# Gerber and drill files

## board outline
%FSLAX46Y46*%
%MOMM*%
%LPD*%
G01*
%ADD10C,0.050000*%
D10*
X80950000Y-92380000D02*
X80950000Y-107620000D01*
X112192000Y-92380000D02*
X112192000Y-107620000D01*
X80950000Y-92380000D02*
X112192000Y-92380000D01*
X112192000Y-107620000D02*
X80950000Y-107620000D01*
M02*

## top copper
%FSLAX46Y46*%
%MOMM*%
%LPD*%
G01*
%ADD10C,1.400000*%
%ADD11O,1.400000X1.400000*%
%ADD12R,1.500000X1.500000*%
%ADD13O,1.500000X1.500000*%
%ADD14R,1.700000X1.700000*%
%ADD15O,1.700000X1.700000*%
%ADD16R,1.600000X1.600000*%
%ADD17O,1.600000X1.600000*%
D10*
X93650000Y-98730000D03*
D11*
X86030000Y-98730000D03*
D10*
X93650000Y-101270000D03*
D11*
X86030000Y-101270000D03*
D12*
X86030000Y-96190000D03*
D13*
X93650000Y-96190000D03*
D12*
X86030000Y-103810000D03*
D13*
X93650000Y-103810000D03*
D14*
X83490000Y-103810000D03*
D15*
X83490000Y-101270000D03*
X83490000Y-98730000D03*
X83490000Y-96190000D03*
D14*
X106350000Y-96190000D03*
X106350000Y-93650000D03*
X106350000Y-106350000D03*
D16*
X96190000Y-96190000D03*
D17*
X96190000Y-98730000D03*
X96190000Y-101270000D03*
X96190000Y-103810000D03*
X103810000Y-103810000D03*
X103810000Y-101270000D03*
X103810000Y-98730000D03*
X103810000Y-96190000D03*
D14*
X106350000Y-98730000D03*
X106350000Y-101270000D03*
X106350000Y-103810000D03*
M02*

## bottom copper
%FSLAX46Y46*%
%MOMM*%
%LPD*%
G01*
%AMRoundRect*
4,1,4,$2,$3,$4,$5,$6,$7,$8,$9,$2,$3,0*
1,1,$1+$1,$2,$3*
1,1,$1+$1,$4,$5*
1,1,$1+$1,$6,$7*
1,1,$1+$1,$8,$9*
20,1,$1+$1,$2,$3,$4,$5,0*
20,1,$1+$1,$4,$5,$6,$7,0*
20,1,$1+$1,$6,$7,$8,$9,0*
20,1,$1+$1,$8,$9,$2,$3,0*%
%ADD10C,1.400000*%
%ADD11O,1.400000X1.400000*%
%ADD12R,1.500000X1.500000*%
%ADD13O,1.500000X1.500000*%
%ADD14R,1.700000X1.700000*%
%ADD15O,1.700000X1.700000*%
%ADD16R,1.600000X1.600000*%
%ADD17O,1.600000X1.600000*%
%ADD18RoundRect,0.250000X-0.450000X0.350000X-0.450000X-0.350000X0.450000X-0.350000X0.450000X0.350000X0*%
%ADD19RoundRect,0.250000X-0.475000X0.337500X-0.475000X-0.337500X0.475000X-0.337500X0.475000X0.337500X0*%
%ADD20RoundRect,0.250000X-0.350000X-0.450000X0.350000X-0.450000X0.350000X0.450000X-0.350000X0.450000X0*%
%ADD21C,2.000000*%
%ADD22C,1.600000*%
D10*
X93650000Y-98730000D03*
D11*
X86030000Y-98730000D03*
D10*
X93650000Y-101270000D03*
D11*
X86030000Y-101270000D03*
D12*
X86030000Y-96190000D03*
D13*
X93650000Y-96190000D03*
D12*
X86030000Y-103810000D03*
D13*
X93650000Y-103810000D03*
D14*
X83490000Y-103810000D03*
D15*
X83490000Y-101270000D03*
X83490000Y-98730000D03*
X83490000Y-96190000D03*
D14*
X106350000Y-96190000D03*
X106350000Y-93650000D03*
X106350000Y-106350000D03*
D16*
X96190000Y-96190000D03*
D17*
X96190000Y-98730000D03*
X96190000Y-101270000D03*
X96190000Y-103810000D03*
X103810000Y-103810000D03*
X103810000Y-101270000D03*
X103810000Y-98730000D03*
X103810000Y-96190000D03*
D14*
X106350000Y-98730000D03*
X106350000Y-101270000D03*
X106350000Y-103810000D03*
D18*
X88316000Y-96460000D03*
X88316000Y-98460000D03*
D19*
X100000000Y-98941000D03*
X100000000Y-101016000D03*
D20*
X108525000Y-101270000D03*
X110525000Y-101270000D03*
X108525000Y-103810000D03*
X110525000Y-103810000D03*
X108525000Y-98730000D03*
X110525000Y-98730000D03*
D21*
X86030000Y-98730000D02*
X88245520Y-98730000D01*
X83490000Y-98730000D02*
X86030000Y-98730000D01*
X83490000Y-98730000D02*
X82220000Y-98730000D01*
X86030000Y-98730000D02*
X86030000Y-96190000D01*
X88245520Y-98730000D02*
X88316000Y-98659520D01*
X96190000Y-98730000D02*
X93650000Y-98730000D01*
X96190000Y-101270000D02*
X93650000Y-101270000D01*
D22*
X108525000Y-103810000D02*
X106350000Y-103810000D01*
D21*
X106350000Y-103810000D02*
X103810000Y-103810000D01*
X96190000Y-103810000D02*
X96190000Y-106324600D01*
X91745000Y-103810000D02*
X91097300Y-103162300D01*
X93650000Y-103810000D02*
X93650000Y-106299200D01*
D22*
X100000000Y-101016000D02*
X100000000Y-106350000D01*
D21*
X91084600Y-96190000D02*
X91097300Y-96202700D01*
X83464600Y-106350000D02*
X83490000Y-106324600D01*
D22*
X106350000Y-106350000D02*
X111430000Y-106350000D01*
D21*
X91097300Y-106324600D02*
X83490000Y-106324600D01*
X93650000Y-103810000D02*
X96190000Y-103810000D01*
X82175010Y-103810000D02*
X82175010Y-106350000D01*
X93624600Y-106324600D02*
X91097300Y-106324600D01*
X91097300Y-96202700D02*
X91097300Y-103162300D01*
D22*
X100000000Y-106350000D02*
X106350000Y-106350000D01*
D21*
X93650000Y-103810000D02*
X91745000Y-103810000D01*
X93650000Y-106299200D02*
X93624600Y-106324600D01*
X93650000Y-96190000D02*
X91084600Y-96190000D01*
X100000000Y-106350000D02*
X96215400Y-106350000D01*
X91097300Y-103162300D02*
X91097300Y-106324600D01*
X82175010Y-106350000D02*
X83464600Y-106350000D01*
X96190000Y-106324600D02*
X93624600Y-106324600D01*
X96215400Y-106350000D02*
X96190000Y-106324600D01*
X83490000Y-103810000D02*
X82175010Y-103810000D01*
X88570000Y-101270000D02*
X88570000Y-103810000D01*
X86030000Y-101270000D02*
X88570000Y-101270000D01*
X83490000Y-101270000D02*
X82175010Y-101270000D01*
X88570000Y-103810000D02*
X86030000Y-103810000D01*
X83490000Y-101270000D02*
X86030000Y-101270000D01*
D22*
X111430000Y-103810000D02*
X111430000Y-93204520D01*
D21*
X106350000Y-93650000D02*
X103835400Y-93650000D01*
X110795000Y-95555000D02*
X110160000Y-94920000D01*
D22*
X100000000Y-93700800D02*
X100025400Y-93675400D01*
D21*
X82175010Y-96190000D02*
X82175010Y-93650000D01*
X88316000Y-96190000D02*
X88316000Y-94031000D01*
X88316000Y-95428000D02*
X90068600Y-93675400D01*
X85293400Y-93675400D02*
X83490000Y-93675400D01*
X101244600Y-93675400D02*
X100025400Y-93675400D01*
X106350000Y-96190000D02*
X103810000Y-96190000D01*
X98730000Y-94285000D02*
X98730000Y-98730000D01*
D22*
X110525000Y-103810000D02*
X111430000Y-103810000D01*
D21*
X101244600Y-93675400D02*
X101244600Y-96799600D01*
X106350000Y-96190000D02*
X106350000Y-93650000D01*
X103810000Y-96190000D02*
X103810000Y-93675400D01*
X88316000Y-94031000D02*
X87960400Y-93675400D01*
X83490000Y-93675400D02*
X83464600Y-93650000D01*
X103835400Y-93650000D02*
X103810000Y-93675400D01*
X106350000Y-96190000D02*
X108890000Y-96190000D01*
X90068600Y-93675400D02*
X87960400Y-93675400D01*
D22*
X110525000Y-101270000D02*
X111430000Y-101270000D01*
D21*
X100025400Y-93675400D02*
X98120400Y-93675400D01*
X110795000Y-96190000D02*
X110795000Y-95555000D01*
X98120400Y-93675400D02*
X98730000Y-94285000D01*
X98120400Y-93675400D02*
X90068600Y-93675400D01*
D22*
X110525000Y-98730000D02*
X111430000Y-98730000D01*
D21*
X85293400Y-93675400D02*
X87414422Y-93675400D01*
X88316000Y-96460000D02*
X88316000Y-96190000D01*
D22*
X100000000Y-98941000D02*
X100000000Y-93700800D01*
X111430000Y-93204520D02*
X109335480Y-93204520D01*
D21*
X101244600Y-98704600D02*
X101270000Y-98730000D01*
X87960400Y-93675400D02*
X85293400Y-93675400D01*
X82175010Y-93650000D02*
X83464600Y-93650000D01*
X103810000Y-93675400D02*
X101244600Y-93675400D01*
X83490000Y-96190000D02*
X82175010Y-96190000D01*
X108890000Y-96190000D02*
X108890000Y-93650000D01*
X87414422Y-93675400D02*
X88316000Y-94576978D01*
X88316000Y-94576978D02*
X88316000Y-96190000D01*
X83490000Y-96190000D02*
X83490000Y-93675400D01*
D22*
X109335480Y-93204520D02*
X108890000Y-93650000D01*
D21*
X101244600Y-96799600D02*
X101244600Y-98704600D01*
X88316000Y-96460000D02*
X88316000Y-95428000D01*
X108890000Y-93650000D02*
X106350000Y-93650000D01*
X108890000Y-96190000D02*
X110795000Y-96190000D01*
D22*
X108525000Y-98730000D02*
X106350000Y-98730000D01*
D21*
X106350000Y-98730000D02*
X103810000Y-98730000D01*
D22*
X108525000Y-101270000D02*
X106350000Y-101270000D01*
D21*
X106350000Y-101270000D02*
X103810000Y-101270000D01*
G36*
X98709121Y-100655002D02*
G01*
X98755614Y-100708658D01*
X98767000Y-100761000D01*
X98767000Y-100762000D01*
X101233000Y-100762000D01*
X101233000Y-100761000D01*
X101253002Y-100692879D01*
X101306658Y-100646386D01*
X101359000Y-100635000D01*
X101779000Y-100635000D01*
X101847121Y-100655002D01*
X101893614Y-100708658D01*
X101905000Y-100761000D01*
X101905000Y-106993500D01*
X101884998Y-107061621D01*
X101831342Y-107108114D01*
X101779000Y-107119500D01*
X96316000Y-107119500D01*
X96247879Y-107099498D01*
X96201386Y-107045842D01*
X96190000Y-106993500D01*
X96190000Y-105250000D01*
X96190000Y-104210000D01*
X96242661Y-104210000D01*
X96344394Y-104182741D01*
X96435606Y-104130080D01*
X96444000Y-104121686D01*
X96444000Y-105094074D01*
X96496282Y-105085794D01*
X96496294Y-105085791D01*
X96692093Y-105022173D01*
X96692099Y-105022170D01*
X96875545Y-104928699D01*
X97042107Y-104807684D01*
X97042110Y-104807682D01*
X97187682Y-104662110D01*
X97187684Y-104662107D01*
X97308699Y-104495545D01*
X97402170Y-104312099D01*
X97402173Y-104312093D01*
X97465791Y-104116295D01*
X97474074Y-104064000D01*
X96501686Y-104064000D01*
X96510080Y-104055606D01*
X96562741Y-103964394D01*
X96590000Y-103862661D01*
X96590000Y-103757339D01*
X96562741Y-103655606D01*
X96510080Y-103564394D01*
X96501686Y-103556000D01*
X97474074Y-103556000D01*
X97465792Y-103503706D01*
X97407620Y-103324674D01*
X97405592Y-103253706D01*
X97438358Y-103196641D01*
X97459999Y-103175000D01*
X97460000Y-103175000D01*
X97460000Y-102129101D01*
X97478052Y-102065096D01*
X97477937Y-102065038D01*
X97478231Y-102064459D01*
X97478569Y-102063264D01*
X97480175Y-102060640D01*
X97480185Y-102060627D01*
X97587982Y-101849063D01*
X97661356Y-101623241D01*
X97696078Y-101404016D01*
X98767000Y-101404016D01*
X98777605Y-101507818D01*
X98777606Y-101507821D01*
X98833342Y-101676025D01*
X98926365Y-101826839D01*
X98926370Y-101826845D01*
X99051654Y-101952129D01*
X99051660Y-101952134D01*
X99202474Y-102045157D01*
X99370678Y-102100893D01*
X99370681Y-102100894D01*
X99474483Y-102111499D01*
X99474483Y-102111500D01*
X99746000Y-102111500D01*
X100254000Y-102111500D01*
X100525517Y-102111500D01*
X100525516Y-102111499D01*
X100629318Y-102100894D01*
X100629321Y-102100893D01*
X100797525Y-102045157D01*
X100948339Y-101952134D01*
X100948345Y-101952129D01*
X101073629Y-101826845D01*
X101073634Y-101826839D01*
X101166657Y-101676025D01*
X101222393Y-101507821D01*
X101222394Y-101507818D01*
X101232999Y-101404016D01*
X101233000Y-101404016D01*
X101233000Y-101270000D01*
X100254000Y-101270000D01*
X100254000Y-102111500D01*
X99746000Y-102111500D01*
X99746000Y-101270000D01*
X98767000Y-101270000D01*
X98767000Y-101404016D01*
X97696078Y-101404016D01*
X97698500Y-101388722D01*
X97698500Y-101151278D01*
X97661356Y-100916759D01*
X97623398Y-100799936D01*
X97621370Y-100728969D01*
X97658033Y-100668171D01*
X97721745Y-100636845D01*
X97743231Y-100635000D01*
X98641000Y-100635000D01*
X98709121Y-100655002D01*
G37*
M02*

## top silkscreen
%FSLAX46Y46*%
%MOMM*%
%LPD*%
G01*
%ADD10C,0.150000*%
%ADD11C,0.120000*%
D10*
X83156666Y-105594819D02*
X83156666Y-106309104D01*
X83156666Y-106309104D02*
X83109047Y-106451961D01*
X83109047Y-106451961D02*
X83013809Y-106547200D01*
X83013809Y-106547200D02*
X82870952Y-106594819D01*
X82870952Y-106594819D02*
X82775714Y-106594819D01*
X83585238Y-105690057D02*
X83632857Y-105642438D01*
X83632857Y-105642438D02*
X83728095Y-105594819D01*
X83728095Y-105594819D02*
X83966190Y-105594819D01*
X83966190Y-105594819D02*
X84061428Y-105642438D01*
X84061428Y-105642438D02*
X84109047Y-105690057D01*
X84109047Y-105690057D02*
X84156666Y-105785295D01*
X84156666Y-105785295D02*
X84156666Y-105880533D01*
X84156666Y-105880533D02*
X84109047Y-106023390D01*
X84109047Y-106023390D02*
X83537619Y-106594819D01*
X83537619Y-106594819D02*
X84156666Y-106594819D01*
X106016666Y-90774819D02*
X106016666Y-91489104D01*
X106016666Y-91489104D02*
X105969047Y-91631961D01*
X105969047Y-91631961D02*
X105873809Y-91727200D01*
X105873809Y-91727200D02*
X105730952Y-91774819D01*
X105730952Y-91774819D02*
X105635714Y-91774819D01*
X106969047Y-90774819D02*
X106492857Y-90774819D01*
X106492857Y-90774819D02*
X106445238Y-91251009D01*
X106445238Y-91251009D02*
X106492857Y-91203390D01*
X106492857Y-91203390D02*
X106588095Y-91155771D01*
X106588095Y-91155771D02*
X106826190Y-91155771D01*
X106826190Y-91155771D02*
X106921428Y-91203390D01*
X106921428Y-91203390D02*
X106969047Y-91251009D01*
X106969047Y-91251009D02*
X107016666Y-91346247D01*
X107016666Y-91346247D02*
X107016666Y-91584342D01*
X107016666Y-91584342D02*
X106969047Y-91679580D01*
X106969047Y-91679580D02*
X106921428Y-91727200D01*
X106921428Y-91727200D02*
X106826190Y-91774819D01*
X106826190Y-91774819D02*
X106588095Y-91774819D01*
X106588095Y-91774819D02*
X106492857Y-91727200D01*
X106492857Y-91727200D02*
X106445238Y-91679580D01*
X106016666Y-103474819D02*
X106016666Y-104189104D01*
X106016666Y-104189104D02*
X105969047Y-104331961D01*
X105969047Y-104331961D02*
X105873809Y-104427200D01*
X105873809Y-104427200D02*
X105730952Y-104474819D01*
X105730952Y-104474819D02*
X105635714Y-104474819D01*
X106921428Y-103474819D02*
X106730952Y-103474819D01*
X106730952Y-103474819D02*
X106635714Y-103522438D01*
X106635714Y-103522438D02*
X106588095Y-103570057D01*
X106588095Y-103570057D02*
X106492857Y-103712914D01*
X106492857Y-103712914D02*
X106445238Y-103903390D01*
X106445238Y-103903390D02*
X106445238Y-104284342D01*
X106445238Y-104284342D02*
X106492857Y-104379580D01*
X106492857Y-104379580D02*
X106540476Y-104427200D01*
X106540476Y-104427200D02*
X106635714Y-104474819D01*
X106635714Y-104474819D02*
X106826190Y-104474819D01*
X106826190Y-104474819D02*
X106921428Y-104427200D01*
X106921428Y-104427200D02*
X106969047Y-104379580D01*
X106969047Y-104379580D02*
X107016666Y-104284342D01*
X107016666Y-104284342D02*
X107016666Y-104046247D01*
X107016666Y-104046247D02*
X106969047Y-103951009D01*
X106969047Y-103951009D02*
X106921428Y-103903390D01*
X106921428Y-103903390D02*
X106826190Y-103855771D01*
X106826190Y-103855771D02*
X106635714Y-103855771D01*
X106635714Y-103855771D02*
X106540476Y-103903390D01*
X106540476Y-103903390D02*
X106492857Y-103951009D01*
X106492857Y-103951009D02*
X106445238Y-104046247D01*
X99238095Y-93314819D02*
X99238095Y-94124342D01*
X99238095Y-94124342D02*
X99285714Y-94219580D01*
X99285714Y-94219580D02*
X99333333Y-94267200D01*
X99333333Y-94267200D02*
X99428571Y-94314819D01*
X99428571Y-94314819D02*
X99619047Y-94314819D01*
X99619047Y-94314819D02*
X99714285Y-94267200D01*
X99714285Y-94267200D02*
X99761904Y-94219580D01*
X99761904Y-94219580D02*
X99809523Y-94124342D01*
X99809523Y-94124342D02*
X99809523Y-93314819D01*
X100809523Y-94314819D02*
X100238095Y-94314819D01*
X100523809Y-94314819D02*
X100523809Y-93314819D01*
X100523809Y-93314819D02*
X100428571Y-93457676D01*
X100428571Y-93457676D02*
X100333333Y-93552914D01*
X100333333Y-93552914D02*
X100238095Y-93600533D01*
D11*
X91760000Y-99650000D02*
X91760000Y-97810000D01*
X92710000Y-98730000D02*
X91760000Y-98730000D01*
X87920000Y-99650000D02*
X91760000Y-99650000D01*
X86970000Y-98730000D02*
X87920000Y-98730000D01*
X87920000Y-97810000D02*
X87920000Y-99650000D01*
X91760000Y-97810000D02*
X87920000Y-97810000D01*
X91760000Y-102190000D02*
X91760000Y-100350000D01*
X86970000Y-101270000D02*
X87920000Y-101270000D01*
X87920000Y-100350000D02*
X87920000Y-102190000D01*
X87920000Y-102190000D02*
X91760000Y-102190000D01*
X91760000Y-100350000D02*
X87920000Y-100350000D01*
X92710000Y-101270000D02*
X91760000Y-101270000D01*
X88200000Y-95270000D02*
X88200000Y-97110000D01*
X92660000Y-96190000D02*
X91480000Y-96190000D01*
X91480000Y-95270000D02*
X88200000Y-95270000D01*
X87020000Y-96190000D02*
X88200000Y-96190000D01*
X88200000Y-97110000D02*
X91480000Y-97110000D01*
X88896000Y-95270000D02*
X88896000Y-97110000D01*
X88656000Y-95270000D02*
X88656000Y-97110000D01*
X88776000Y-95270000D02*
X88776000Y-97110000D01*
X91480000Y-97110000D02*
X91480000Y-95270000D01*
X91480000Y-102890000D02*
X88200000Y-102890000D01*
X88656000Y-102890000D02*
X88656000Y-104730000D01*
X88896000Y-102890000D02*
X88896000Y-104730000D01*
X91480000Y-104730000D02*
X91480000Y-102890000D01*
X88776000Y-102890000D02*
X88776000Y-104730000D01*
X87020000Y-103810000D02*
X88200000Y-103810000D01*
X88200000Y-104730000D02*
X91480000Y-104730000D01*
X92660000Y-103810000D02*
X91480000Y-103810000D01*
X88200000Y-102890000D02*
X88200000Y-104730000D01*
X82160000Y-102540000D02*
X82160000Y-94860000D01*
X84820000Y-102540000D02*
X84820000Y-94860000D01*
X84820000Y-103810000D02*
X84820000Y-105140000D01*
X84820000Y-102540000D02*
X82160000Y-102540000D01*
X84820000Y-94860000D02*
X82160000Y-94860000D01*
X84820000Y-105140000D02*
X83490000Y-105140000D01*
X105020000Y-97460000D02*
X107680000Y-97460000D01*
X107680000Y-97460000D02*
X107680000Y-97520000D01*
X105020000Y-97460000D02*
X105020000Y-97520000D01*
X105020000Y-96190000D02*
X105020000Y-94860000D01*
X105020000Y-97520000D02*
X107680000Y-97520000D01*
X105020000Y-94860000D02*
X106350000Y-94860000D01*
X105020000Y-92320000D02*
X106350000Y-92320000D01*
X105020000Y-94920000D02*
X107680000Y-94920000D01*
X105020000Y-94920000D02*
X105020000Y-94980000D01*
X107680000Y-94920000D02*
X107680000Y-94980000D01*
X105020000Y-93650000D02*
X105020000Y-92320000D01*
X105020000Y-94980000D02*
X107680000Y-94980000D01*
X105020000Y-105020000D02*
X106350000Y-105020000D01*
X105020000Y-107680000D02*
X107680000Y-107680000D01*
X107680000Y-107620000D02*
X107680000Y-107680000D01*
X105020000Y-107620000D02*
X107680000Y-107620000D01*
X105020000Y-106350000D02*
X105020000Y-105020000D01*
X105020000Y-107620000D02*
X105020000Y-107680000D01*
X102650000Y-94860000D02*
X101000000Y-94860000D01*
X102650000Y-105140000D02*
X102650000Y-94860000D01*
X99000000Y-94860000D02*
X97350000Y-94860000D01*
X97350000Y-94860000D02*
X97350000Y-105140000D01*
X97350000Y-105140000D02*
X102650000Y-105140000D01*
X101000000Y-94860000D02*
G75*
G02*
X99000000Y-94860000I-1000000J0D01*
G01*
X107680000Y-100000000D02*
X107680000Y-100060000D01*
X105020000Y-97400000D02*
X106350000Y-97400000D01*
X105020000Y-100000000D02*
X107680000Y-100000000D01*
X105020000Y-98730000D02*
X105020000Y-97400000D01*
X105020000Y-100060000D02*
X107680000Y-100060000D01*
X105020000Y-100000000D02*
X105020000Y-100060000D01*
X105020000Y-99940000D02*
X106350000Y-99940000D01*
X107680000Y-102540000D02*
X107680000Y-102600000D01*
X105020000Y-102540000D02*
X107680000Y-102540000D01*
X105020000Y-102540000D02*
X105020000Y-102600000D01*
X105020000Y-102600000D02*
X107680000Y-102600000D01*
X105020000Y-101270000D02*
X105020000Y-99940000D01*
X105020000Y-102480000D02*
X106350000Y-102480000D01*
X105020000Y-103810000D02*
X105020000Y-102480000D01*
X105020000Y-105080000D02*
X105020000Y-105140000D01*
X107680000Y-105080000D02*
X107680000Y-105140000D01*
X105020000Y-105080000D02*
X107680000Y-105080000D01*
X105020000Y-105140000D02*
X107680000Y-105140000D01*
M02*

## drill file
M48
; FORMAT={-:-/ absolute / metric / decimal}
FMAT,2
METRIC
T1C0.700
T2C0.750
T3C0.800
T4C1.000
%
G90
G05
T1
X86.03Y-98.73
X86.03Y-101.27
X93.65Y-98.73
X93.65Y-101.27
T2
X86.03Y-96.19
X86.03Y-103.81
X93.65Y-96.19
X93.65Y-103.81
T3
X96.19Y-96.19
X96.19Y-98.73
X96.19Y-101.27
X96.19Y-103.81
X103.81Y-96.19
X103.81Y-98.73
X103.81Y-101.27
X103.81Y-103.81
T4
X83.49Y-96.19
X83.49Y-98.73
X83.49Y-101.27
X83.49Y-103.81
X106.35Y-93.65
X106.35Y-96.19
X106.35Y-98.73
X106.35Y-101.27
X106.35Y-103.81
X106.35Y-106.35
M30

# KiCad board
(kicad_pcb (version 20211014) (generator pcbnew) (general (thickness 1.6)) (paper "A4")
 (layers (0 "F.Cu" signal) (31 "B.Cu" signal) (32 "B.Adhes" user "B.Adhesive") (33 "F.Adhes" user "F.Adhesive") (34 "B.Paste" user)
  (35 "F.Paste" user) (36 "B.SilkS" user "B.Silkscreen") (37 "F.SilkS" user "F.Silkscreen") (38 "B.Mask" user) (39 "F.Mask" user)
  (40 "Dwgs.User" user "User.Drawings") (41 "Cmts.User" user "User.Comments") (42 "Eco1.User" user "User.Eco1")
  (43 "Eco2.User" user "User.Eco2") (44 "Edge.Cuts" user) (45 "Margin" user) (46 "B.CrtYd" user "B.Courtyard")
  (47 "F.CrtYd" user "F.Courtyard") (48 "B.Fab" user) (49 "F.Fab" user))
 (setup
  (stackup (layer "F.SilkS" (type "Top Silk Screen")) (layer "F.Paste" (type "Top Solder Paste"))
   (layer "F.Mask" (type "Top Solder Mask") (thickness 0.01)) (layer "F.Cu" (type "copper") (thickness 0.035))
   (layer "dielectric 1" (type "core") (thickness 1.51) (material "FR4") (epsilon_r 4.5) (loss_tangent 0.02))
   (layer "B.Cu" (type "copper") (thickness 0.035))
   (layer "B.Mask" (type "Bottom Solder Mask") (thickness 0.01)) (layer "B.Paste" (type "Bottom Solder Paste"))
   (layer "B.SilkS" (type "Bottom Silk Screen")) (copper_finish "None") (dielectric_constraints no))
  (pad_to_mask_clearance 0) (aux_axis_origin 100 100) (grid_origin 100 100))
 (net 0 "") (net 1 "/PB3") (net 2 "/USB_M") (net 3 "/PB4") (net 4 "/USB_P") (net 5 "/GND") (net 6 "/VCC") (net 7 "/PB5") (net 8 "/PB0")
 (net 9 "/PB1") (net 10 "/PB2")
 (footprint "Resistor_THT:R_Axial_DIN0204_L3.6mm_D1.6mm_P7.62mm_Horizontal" (layer "F.Cu") (at 93.65 98.73 180)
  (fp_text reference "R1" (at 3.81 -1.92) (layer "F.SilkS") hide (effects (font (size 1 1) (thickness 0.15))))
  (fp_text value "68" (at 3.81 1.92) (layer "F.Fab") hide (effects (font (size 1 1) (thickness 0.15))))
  (fp_line (start 1.89 -0.92) (end 1.89 0.92) (layer "F.SilkS") (width 0.12))
  (fp_line (start 0.94 0) (end 1.89 0) (layer "F.SilkS") (width 0.12))
  (fp_line (start 5.73 -0.92) (end 1.89 -0.92) (layer "F.SilkS") (width 0.12))
  (fp_line (start 6.68 0) (end 5.73 0) (layer "F.SilkS") (width 0.12))
  (fp_line (start 5.73 0.92) (end 5.73 -0.92) (layer "F.SilkS") (width 0.12))
  (fp_line (start 1.89 0.92) (end 5.73 0.92) (layer "F.SilkS") (width 0.12))
  (pad "1" thru_hole circle locked (at 0 0 180) (size 1.4 1.4) (drill 0.7) (layers *.Cu *.Mask) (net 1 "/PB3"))
  (pad "2" thru_hole oval locked (at 7.62 0 180) (size 1.4 1.4) (drill 0.7) (layers *.Cu *.Mask) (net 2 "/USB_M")))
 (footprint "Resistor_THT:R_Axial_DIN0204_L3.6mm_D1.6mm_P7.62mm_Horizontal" (layer "F.Cu") (at 93.65 101.27 180)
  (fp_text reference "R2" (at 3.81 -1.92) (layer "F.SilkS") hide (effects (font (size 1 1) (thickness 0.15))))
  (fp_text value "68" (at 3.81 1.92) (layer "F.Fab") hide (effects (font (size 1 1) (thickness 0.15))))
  (fp_line (start 1.89 -0.92) (end 1.89 0.92) (layer "F.SilkS") (width 0.12))
  (fp_line (start 6.68 0) (end 5.73 0) (layer "F.SilkS") (width 0.12))
  (fp_line (start 5.73 0.92) (end 5.73 -0.92) (layer "F.SilkS") (width 0.12))
  (fp_line (start 5.73 -0.92) (end 1.89 -0.92) (layer "F.SilkS") (width 0.12))
  (fp_line (start 1.89 0.92) (end 5.73 0.92) (layer "F.SilkS") (width 0.12))
  (fp_line (start 0.94 0) (end 1.89 0) (layer "F.SilkS") (width 0.12))
  (pad "1" thru_hole circle locked (at 0 0 180) (size 1.4 1.4) (drill 0.7) (layers *.Cu *.Mask) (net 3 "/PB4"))
  (pad "2" thru_hole oval locked (at 7.62 0 180) (size 1.4 1.4) (drill 0.7) (layers *.Cu *.Mask) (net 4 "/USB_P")))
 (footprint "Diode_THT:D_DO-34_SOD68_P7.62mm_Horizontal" (layer "F.Cu") (at 86.03 96.19)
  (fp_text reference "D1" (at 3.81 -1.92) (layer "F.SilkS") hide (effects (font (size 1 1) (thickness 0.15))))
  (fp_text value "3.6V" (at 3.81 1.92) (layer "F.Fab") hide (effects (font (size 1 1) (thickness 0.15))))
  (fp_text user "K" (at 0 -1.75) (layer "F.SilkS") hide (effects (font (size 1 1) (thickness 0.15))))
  (fp_line (start 2.17 -0.92) (end 2.17 0.92) (layer "F.SilkS") (width 0.12))
  (fp_line (start 6.63 0) (end 5.45 0) (layer "F.SilkS") (width 0.12))
  (fp_line (start 5.45 -0.92) (end 2.17 -0.92) (layer "F.SilkS") (width 0.12))
  (fp_line (start 0.99 0) (end 2.17 0) (layer "F.SilkS") (width 0.12))
  (fp_line (start 2.17 0.92) (end 5.45 0.92) (layer "F.SilkS") (width 0.12))
  (fp_line (start 2.866 -0.92) (end 2.866 0.92) (layer "F.SilkS") (width 0.12))
  (fp_line (start 2.626 -0.92) (end 2.626 0.92) (layer "F.SilkS") (width 0.12))
  (fp_line (start 2.746 -0.92) (end 2.746 0.92) (layer "F.SilkS") (width 0.12))
  (fp_line (start 5.45 0.92) (end 5.45 -0.92) (layer "F.SilkS") (width 0.12))
  (pad "1" thru_hole rect locked (at 0 0) (size 1.5 1.5) (drill 0.75) (layers *.Cu *.Mask) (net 2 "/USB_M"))
  (pad "2" thru_hole oval locked (at 7.62 0) (size 1.5 1.5) (drill 0.75) (layers *.Cu *.Mask) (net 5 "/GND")))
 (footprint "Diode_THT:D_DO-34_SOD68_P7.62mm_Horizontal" (layer "F.Cu") (at 86.03 103.81)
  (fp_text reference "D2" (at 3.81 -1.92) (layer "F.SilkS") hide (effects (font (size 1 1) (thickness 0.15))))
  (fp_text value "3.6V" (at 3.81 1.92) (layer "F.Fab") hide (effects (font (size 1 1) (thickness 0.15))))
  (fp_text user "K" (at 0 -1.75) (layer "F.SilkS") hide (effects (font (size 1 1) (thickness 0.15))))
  (fp_line (start 5.45 -0.92) (end 2.17 -0.92) (layer "F.SilkS") (width 0.12))
  (fp_line (start 2.626 -0.92) (end 2.626 0.92) (layer "F.SilkS") (width 0.12))
  (fp_line (start 2.866 -0.92) (end 2.866 0.92) (layer "F.SilkS") (width 0.12))
  (fp_line (start 5.45 0.92) (end 5.45 -0.92) (layer "F.SilkS") (width 0.12))
  (fp_line (start 2.746 -0.92) (end 2.746 0.92) (layer "F.SilkS") (width 0.12))
  (fp_line (start 0.99 0) (end 2.17 0) (layer "F.SilkS") (width 0.12))
  (fp_line (start 2.17 0.92) (end 5.45 0.92) (layer "F.SilkS") (width 0.12))
  (fp_line (start 6.63 0) (end 5.45 0) (layer "F.SilkS") (width 0.12))
  (fp_line (start 2.17 -0.92) (end 2.17 0.92) (layer "F.SilkS") (width 0.12))
  (pad "1" thru_hole rect locked (at 0 0) (size 1.5 1.5) (drill 0.75) (layers *.Cu *.Mask) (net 4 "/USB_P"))
  (pad "2" thru_hole oval locked (at 7.62 0) (size 1.5 1.5) (drill 0.75) (layers *.Cu *.Mask) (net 5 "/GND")))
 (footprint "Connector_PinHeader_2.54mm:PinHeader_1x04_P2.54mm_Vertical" (layer "F.Cu") (at 83.49 103.81 180)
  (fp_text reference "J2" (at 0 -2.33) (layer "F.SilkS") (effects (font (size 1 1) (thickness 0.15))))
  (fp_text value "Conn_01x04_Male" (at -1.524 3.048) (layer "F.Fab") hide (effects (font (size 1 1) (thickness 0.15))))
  (fp_line (start 1.33 1.27) (end 1.33 8.95) (layer "F.SilkS") (width 0.12))
  (fp_line (start -1.33 1.27) (end -1.33 8.95) (layer "F.SilkS") (width 0.12))
  (fp_line (start -1.33 0) (end -1.33 -1.33) (layer "F.SilkS") (width 0.12))
  (fp_line (start -1.33 1.27) (end 1.33 1.27) (layer "F.SilkS") (width 0.12))
  (fp_line (start -1.33 8.95) (end 1.33 8.95) (layer "F.SilkS") (width 0.12))
  (fp_line (start -1.33 -1.33) (end 0 -1.33) (layer "F.SilkS") (width 0.12))
  (pad "1" thru_hole rect locked (at 0 0 180) (size 1.7 1.7) (drill 1) (layers *.Cu *.Mask) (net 5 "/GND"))
  (pad "2" thru_hole oval locked (at 0 2.54 180) (size 1.7 1.7) (drill 1) (layers *.Cu *.Mask) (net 4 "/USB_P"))
  (pad "3" thru_hole oval locked (at 0 5.08 180) (size 1.7 1.7) (drill 1) (layers *.Cu *.Mask) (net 2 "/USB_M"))
  (pad "4" thru_hole oval locked (at 0 7.62 180) (size 1.7 1.7) (drill 1) (layers *.Cu *.Mask) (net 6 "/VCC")))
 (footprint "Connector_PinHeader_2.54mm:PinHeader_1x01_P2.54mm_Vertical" (layer "F.Cu") (at 106.35 96.19)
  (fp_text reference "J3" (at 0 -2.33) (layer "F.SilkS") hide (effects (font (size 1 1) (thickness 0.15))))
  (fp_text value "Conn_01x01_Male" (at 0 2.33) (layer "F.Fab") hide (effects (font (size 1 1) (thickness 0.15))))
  (fp_line (start -1.33 1.27) (end 1.33 1.27) (layer "F.SilkS") (width 0.12))
  (fp_line (start 1.33 1.27) (end 1.33 1.33) (layer "F.SilkS") (width 0.12))
  (fp_line (start -1.33 1.27) (end -1.33 1.33) (layer "F.SilkS") (width 0.12))
  (fp_line (start -1.33 0) (end -1.33 -1.33) (layer "F.SilkS") (width 0.12))
  (fp_line (start -1.33 1.33) (end 1.33 1.33) (layer "F.SilkS") (width 0.12))
  (fp_line (start -1.33 -1.33) (end 0 -1.33) (layer "F.SilkS") (width 0.12))
  (pad "1" thru_hole rect locked (at 0 0) (size 1.7 1.7) (drill 1) (layers *.Cu *.Mask) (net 6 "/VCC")))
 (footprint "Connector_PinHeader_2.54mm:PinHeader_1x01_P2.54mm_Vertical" (layer "F.Cu") (at 106.35 93.65)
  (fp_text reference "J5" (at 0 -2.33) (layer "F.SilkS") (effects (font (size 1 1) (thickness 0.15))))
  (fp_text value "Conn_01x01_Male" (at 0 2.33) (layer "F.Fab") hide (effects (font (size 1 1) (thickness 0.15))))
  (fp_line (start -1.33 -1.33) (end 0 -1.33) (layer "F.SilkS") (width 0.12))
  (fp_line (start -1.33 1.27) (end 1.33 1.27) (layer "F.SilkS") (width 0.12))
  (fp_line (start -1.33 1.27) (end -1.33 1.33) (layer "F.SilkS") (width 0.12))
  (fp_line (start 1.33 1.27) (end 1.33 1.33) (layer "F.SilkS") (width 0.12))
  (fp_line (start -1.33 0) (end -1.33 -1.33) (layer "F.SilkS") (width 0.12))
  (fp_line (start -1.33 1.33) (end 1.33 1.33) (layer "F.SilkS") (width 0.12))
  (pad "1" thru_hole rect locked (at 0 0) (size 1.7 1.7) (drill 1) (layers *.Cu *.Mask) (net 6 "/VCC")))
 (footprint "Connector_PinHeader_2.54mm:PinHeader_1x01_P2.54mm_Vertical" (layer "F.Cu") (at 106.35 106.35)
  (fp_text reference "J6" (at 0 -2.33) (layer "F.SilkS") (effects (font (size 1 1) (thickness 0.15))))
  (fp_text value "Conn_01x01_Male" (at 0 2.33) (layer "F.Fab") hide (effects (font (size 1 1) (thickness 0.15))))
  (fp_line (start -1.33 -1.33) (end 0 -1.33) (layer "F.SilkS") (width 0.12))
  (fp_line (start -1.33 1.33) (end 1.33 1.33) (layer "F.SilkS") (width 0.12))
  (fp_line (start 1.33 1.27) (end 1.33 1.33) (layer "F.SilkS") (width 0.12))
  (fp_line (start -1.33 1.27) (end 1.33 1.27) (layer "F.SilkS") (width 0.12))
  (fp_line (start -1.33 0) (end -1.33 -1.33) (layer "F.SilkS") (width 0.12))
  (fp_line (start -1.33 1.27) (end -1.33 1.33) (layer "F.SilkS") (width 0.12))
  (pad "1" thru_hole rect locked (at 0 0) (size 1.7 1.7) (drill 1) (layers *.Cu *.Mask) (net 5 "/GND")))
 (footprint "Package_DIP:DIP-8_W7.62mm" (layer "F.Cu") (at 96.19 96.19)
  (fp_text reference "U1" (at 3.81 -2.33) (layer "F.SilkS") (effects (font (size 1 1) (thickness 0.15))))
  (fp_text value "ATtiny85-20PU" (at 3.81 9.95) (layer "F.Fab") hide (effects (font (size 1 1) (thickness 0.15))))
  (fp_line (start 6.46 -1.33) (end 4.81 -1.33) (layer "F.SilkS") (width 0.12))
  (fp_line (start 6.46 8.95) (end 6.46 -1.33) (layer "F.SilkS") (width 0.12))
  (fp_line (start 2.81 -1.33) (end 1.16 -1.33) (layer "F.SilkS") (width 0.12))
  (fp_line (start 1.16 -1.33) (end 1.16 8.95) (layer "F.SilkS") (width 0.12))
  (fp_line (start 1.16 8.95) (end 6.46 8.95) (layer "F.SilkS") (width 0.12))
  (fp_arc (start 4.81 -1.33) (mid 3.81 -0.33) (end 2.81 -1.33) (layer "F.SilkS") (width 0.12))
  (pad "1" thru_hole rect locked (at 0 0) (size 1.6 1.6) (drill 0.8) (layers *.Cu *.Mask) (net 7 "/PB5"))
  (pad "2" thru_hole oval locked (at 0 2.54) (size 1.6 1.6) (drill 0.8) (layers *.Cu *.Mask) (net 1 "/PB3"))
  (pad "3" thru_hole oval locked (at 0 5.08) (size 1.6 1.6) (drill 0.8) (layers *.Cu *.Mask) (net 3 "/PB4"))
  (pad "4" thru_hole oval locked (at 0 7.62) (size 1.6 1.6) (drill 0.8) (layers *.Cu *.Mask) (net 5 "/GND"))
  (pad "5" thru_hole oval locked (at 7.62 7.62) (size 1.6 1.6) (drill 0.8) (layers *.Cu *.Mask) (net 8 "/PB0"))
  (pad "6" thru_hole oval locked (at 7.62 5.08) (size 1.6 1.6) (drill 0.8) (layers *.Cu *.Mask) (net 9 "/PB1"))
  (pad "7" thru_hole oval locked (at 7.62 2.54) (size 1.6 1.6) (drill 0.8) (layers *.Cu *.Mask) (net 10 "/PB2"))
  (pad "8" thru_hole oval locked (at 7.62 0) (size 1.6 1.6) (drill 0.8) (layers *.Cu *.Mask) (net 6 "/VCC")))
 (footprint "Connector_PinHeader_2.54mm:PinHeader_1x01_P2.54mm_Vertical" (layer "F.Cu") (at 106.35 98.73)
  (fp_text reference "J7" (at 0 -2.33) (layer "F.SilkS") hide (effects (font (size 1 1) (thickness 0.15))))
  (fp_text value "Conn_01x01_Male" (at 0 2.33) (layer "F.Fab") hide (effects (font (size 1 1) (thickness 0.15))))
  (fp_line (start 1.33 1.27) (end 1.33 1.33) (layer "F.SilkS") (width 0.12))
  (fp_line (start -1.33 -1.33) (end 0 -1.33) (layer "F.SilkS") (width 0.12))
  (fp_line (start -1.33 1.27) (end 1.33 1.27) (layer "F.SilkS") (width 0.12))
  (fp_line (start -1.33 0) (end -1.33 -1.33) (layer "F.SilkS") (width 0.12))
  (fp_line (start -1.33 1.33) (end 1.33 1.33) (layer "F.SilkS") (width 0.12))
  (fp_line (start -1.33 1.27) (end -1.33 1.33) (layer "F.SilkS") (width 0.12))
  (pad "1" thru_hole rect (at 0 0) (size 1.7 1.7) (drill 1) (layers *.Cu *.Mask) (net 10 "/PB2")))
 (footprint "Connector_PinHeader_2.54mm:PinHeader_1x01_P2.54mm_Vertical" (layer "F.Cu") (at 106.35 101.27)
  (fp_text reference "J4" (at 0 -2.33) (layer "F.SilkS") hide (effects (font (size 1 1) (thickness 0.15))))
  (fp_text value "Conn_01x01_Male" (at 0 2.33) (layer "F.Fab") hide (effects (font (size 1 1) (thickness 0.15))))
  (fp_line (start -1.33 -1.33) (end 0 -1.33) (layer "F.SilkS") (width 0.12))
  (fp_line (start 1.33 1.27) (end 1.33 1.33) (layer "F.SilkS") (width 0.12))
  (fp_line (start -1.33 1.27) (end 1.33 1.27) (layer "F.SilkS") (width 0.12))
  (fp_line (start -1.33 1.27) (end -1.33 1.33) (layer "F.SilkS") (width 0.12))
  (fp_line (start -1.33 1.33) (end 1.33 1.33) (layer "F.SilkS") (width 0.12))
  (fp_line (start -1.33 0) (end -1.33 -1.33) (layer "F.SilkS") (width 0.12))
  (pad "1" thru_hole rect (at 0 0) (size 1.7 1.7) (drill 1) (layers *.Cu *.Mask) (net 9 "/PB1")))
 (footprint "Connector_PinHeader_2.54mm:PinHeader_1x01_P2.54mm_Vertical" (layer "F.Cu") (at 106.35 103.81)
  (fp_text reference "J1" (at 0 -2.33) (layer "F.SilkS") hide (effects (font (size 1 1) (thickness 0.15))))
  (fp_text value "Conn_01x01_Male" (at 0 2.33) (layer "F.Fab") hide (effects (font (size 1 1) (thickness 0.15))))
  (fp_line (start -1.33 -1.33) (end 0 -1.33) (layer "F.SilkS") (width 0.12))
  (fp_line (start -1.33 0) (end -1.33 -1.33) (layer "F.SilkS") (width 0.12))
  (fp_line (start -1.33 1.27) (end -1.33 1.33) (layer "F.SilkS") (width 0.12))
  (fp_line (start 1.33 1.27) (end 1.33 1.33) (layer "F.SilkS") (width 0.12))
  (fp_line (start -1.33 1.27) (end 1.33 1.27) (layer "F.SilkS") (width 0.12))
  (fp_line (start -1.33 1.33) (end 1.33 1.33) (layer "F.SilkS") (width 0.12))
  (pad "1" thru_hole rect (at 0 0) (size 1.7 1.7) (drill 1) (layers *.Cu *.Mask) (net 8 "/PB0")))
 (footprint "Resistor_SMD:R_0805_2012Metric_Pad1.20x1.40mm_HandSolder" (layer "B.Cu") (at 88.316 97.46 -90)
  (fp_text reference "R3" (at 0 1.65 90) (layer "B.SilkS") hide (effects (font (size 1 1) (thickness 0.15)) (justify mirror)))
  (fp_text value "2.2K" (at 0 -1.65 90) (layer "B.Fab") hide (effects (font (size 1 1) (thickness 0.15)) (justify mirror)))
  (pad "1" smd roundrect locked (at -1 0 270) (size 1.2 1.4) (layers "B.Cu" "B.Paste" "B.Mask") (roundrect_rratio 0.2083333333)
   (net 6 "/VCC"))
  (pad "2" smd roundrect locked (at 1 0 270) (size 1.2 1.4) (layers "B.Cu" "B.Paste" "B.Mask") (roundrect_rratio 0.2083333333)
   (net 2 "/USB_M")))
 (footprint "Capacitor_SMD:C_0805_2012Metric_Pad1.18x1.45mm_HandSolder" (layer "B.Cu") (at 100 99.9785 -90)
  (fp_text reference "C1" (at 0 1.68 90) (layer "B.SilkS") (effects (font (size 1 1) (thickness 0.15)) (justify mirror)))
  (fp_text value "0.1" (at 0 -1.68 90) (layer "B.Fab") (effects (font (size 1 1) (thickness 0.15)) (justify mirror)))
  (pad "1" smd roundrect locked (at -1.0375 0 270) (size 1.175 1.45) (layers "B.Cu" "B.Paste" "B.Mask") (roundrect_rratio 0.2127659574)
   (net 6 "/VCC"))
  (pad "2" smd roundrect locked (at 1.0375 0 270) (size 1.175 1.45) (layers "B.Cu" "B.Paste" "B.Mask") (roundrect_rratio 0.2127659574)
   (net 5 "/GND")))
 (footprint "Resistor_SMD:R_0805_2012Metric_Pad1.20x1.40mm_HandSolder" (layer "B.Cu") (at 109.525 101.27)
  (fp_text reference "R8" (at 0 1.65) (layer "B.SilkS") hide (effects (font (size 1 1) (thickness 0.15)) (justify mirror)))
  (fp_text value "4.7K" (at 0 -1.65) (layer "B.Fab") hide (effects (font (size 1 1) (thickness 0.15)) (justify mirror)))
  (pad "1" smd roundrect (at -1 0) (size 1.2 1.4) (layers "B.Cu" "B.Paste" "B.Mask") (roundrect_rratio 0.2083333333) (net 9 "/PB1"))
  (pad "2" smd roundrect (at 1 0) (size 1.2 1.4) (layers "B.Cu" "B.Paste" "B.Mask") (roundrect_rratio 0.2083333333) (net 6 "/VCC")))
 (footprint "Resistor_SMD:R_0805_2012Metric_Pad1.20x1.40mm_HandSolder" (layer "B.Cu") (at 109.525 103.81)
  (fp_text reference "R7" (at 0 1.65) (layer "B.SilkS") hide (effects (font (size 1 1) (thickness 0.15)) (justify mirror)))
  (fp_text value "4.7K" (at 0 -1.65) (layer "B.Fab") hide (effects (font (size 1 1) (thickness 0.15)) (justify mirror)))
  (pad "1" smd roundrect (at -1 0) (size 1.2 1.4) (layers "B.Cu" "B.Paste" "B.Mask") (roundrect_rratio 0.2083333333) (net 8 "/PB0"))
  (pad "2" smd roundrect (at 1 0) (size 1.2 1.4) (layers "B.Cu" "B.Paste" "B.Mask") (roundrect_rratio 0.2083333333) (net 6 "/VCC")))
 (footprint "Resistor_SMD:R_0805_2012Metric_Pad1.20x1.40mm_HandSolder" (layer "B.Cu") (at 109.525 98.73)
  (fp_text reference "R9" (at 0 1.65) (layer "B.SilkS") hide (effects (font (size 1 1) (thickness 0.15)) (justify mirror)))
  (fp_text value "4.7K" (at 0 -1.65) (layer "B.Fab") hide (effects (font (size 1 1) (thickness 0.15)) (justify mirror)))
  (pad "1" smd roundrect (at -1 0) (size 1.2 1.4) (layers "B.Cu" "B.Paste" "B.Mask") (roundrect_rratio 0.2083333333) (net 10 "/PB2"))
  (pad "2" smd roundrect (at 1 0) (size 1.2 1.4) (layers "B.Cu" "B.Paste" "B.Mask") (roundrect_rratio 0.2083333333) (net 6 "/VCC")))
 (gr_line (start 80.95 92.38) (end 80.95 107.62) (layer "Edge.Cuts") (width 0.05))
 (gr_line (start 112.192 92.38) (end 112.192 107.62) (layer "Edge.Cuts") (width 0.05))
 (gr_line (start 80.95 92.38) (end 112.192 92.38) (layer "Edge.Cuts") (width 0.05))
 (gr_line (start 112.192 107.62) (end 80.95 107.62) (layer "Edge.Cuts") (width 0.05))
 (segment (start 86.03 98.73) (end 88.24552 98.73) (width 2) (layer "B.Cu") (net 2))
 (segment (start 83.49 98.73) (end 86.03 98.73) (width 2) (layer "B.Cu") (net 2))
 (segment (start 83.49 98.73) (end 82.22 98.73) (width 2) (layer "B.Cu") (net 2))
 (segment (start 86.03 98.73) (end 86.03 96.19) (width 2) (layer "B.Cu") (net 2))
 (segment (start 88.24552 98.73) (end 88.316 98.65952) (width 2) (layer "B.Cu") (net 2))
 (segment (start 96.19 98.73) (end 93.65 98.73) (width 2) (layer "B.Cu") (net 1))
 (segment (start 96.19 101.27) (end 93.65 101.27) (width 2) (layer "B.Cu") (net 3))
 (segment (start 108.525 103.81) (end 106.35 103.81) (width 1.6) (layer "B.Cu") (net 8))
 (segment (start 106.35 103.81) (end 103.81 103.81) (width 2) (layer "B.Cu") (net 8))
 (segment (start 96.19 103.81) (end 96.19 106.3246) (width 2) (layer "B.Cu") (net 5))
 (segment (start 91.745 103.81) (end 91.0973 103.1623) (width 2) (layer "B.Cu") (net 5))
 (segment (start 93.65 103.81) (end 93.65 106.2992) (width 2) (layer "B.Cu") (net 5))
 (segment (start 100 101.016) (end 100 106.35) (width 1.6) (layer "B.Cu") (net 5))
 (segment (start 91.0846 96.19) (end 91.0973 96.2027) (width 2) (layer "B.Cu") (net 5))
 (segment (start 83.4646 106.35) (end 83.49 106.3246) (width 2) (layer "B.Cu") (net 5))
 (segment (start 106.35 106.35) (end 111.43 106.35) (width 1.6) (layer "B.Cu") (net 5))
 (segment (start 91.0973 106.3246) (end 83.49 106.3246) (width 2) (layer "B.Cu") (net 5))
 (segment (start 93.65 103.81) (end 96.19 103.81) (width 2) (layer "B.Cu") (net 5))
 (segment (start 82.17501 103.81) (end 82.17501 106.35) (width 2) (layer "B.Cu") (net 5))
 (segment (start 93.6246 106.3246) (end 91.0973 106.3246) (width 2) (layer "B.Cu") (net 5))
 (segment (start 91.0973 96.2027) (end 91.0973 103.1623) (width 2) (layer "B.Cu") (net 5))
 (segment (start 100 106.35) (end 106.35 106.35) (width 1.6) (layer "B.Cu") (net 5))
 (segment (start 93.65 103.81) (end 91.745 103.81) (width 2) (layer "B.Cu") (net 5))
 (segment (start 93.65 106.2992) (end 93.6246 106.3246) (width 2) (layer "B.Cu") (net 5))
 (segment (start 93.65 96.19) (end 91.0846 96.19) (width 2) (layer "B.Cu") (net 5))
 (segment (start 100 106.35) (end 96.2154 106.35) (width 2) (layer "B.Cu") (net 5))
 (segment (start 91.0973 103.1623) (end 91.0973 106.3246) (width 2) (layer "B.Cu") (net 5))
 (segment (start 82.17501 106.35) (end 83.4646 106.35) (width 2) (layer "B.Cu") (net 5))
 (segment (start 96.19 106.3246) (end 93.6246 106.3246) (width 2) (layer "B.Cu") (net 5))
 (segment (start 96.2154 106.35) (end 96.19 106.3246) (width 2) (layer "B.Cu") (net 5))
 (segment (start 83.49 103.81) (end 82.17501 103.81) (width 2) (layer "B.Cu") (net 5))
 (segment (start 88.57 101.27) (end 88.57 103.81) (width 2) (layer "B.Cu") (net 4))
 (segment (start 86.03 101.27) (end 88.57 101.27) (width 2) (layer "B.Cu") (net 4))
 (segment (start 83.49 101.27) (end 82.17501 101.27) (width 2) (layer "B.Cu") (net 4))
 (segment (start 88.57 103.81) (end 86.03 103.81) (width 2) (layer "B.Cu") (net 4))
 (segment (start 83.49 101.27) (end 86.03 101.27) (width 2) (layer "B.Cu") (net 4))
 (segment (start 111.43 103.81) (end 111.43 93.20452) (width 1.6) (layer "B.Cu") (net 6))
 (segment (start 106.35 93.65) (end 103.8354 93.65) (width 2) (layer "B.Cu") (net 6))
 (segment (start 110.795 95.555) (end 110.16 94.92) (width 2) (layer "B.Cu") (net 6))
 (segment (start 100 93.7008) (end 100.0254 93.6754) (width 1.6) (layer "B.Cu") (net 6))
 (segment (start 82.17501 96.19) (end 82.17501 93.65) (width 2) (layer "B.Cu") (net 6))
 (segment (start 88.316 96.19) (end 88.316 94.031) (width 2) (layer "B.Cu") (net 6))
 (segment (start 88.316 95.428) (end 90.0686 93.6754) (width 2) (layer "B.Cu") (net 6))
 (segment (start 85.2934 93.6754) (end 83.49 93.6754) (width 2) (layer "B.Cu") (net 6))
 (segment (start 101.2446 93.6754) (end 100.0254 93.6754) (width 2) (layer "B.Cu") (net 6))
 (segment (start 106.35 96.19) (end 103.81 96.19) (width 2) (layer "B.Cu") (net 6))
 (segment (start 98.73 94.285) (end 98.73 98.73) (width 2) (layer "B.Cu") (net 6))
 (segment (start 110.525 103.81) (end 111.43 103.81) (width 1.6) (layer "B.Cu") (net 6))
 (segment (start 101.2446 93.6754) (end 101.2446 96.7996) (width 2) (layer "B.Cu") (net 6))
 (segment (start 106.35 96.19) (end 106.35 93.65) (width 2) (layer "B.Cu") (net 6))
 (segment (start 103.81 96.19) (end 103.81 93.6754) (width 2) (layer "B.Cu") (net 6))
 (segment (start 88.316 94.031) (end 87.9604 93.6754) (width 2) (layer "B.Cu") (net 6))
 (segment (start 83.49 93.6754) (end 83.4646 93.65) (width 2) (layer "B.Cu") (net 6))
 (segment (start 103.8354 93.65) (end 103.81 93.6754) (width 2) (layer "B.Cu") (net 6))
 (segment (start 106.35 96.19) (end 108.89 96.19) (width 2) (layer "B.Cu") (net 6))
 (segment (start 90.0686 93.6754) (end 87.9604 93.6754) (width 2) (layer "B.Cu") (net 6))
 (segment (start 110.525 101.27) (end 111.43 101.27) (width 1.6) (layer "B.Cu") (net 6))
 (segment (start 100.0254 93.6754) (end 98.1204 93.6754) (width 2) (layer "B.Cu") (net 6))
 (segment (start 110.795 96.19) (end 110.795 95.555) (width 2) (layer "B.Cu") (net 6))
 (segment (start 98.1204 93.6754) (end 98.73 94.285) (width 2) (layer "B.Cu") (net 6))
 (segment (start 98.1204 93.6754) (end 90.0686 93.6754) (width 2) (layer "B.Cu") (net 6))
 (segment (start 110.525 98.73) (end 111.43 98.73) (width 1.6) (layer "B.Cu") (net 6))
 (segment (start 85.2934 93.6754) (end 87.414422 93.6754) (width 2) (layer "B.Cu") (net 6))
 (segment (start 88.316 96.46) (end 88.316 96.19) (width 2) (layer "B.Cu") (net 6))
 (segment (start 100 98.941) (end 100 93.7008) (width 1.6) (layer "B.Cu") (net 6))
 (segment (start 111.43 93.20452) (end 109.33548 93.20452) (width 1.6) (layer "B.Cu") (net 6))
 (segment (start 101.2446 98.7046) (end 101.27 98.73) (width 2) (layer "B.Cu") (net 6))
 (segment (start 87.9604 93.6754) (end 85.2934 93.6754) (width 2) (layer "B.Cu") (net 6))
 (segment (start 82.17501 93.65) (end 83.4646 93.65) (width 2) (layer "B.Cu") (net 6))
 (segment (start 103.81 93.6754) (end 101.2446 93.6754) (width 2) (layer "B.Cu") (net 6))
 (segment (start 83.49 96.19) (end 82.17501 96.19) (width 2) (layer "B.Cu") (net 6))
 (segment (start 108.89 96.19) (end 108.89 93.65) (width 2) (layer "B.Cu") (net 6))
 (segment (start 87.414422 93.6754) (end 88.316 94.576978) (width 2) (layer "B.Cu") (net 6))
 (segment (start 88.316 94.576978) (end 88.316 96.19) (width 2) (layer "B.Cu") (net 6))
 (segment (start 83.49 96.19) (end 83.49 93.6754) (width 2) (layer "B.Cu") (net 6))
 (segment (start 109.33548 93.20452) (end 108.89 93.65) (width 1.6) (layer "B.Cu") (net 6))
 (segment (start 101.2446 96.7996) (end 101.2446 98.7046) (width 2) (layer "B.Cu") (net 6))
 (segment (start 88.316 96.46) (end 88.316 95.428) (width 2) (layer "B.Cu") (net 6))
 (segment (start 108.89 93.65) (end 106.35 93.65) (width 2) (layer "B.Cu") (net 6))
 (segment (start 108.89 96.19) (end 110.795 96.19) (width 2) (layer "B.Cu") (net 6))
 (segment (start 108.525 98.73) (end 106.35 98.73) (width 1.6) (layer "B.Cu") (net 10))
 (segment (start 106.35 98.73) (end 103.81 98.73) (width 2) (layer "B.Cu") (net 10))
 (segment (start 108.525 101.27) (end 106.35 101.27) (width 1.6) (layer "B.Cu") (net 9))
 (segment (start 106.35 101.27) (end 103.81 101.27) (width 2) (layer "B.Cu") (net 9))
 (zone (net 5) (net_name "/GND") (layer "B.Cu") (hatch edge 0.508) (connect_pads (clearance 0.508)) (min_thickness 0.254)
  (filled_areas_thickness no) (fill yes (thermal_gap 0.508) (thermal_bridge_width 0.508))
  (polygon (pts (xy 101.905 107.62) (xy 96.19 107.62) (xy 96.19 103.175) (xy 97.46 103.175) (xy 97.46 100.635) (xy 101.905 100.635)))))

